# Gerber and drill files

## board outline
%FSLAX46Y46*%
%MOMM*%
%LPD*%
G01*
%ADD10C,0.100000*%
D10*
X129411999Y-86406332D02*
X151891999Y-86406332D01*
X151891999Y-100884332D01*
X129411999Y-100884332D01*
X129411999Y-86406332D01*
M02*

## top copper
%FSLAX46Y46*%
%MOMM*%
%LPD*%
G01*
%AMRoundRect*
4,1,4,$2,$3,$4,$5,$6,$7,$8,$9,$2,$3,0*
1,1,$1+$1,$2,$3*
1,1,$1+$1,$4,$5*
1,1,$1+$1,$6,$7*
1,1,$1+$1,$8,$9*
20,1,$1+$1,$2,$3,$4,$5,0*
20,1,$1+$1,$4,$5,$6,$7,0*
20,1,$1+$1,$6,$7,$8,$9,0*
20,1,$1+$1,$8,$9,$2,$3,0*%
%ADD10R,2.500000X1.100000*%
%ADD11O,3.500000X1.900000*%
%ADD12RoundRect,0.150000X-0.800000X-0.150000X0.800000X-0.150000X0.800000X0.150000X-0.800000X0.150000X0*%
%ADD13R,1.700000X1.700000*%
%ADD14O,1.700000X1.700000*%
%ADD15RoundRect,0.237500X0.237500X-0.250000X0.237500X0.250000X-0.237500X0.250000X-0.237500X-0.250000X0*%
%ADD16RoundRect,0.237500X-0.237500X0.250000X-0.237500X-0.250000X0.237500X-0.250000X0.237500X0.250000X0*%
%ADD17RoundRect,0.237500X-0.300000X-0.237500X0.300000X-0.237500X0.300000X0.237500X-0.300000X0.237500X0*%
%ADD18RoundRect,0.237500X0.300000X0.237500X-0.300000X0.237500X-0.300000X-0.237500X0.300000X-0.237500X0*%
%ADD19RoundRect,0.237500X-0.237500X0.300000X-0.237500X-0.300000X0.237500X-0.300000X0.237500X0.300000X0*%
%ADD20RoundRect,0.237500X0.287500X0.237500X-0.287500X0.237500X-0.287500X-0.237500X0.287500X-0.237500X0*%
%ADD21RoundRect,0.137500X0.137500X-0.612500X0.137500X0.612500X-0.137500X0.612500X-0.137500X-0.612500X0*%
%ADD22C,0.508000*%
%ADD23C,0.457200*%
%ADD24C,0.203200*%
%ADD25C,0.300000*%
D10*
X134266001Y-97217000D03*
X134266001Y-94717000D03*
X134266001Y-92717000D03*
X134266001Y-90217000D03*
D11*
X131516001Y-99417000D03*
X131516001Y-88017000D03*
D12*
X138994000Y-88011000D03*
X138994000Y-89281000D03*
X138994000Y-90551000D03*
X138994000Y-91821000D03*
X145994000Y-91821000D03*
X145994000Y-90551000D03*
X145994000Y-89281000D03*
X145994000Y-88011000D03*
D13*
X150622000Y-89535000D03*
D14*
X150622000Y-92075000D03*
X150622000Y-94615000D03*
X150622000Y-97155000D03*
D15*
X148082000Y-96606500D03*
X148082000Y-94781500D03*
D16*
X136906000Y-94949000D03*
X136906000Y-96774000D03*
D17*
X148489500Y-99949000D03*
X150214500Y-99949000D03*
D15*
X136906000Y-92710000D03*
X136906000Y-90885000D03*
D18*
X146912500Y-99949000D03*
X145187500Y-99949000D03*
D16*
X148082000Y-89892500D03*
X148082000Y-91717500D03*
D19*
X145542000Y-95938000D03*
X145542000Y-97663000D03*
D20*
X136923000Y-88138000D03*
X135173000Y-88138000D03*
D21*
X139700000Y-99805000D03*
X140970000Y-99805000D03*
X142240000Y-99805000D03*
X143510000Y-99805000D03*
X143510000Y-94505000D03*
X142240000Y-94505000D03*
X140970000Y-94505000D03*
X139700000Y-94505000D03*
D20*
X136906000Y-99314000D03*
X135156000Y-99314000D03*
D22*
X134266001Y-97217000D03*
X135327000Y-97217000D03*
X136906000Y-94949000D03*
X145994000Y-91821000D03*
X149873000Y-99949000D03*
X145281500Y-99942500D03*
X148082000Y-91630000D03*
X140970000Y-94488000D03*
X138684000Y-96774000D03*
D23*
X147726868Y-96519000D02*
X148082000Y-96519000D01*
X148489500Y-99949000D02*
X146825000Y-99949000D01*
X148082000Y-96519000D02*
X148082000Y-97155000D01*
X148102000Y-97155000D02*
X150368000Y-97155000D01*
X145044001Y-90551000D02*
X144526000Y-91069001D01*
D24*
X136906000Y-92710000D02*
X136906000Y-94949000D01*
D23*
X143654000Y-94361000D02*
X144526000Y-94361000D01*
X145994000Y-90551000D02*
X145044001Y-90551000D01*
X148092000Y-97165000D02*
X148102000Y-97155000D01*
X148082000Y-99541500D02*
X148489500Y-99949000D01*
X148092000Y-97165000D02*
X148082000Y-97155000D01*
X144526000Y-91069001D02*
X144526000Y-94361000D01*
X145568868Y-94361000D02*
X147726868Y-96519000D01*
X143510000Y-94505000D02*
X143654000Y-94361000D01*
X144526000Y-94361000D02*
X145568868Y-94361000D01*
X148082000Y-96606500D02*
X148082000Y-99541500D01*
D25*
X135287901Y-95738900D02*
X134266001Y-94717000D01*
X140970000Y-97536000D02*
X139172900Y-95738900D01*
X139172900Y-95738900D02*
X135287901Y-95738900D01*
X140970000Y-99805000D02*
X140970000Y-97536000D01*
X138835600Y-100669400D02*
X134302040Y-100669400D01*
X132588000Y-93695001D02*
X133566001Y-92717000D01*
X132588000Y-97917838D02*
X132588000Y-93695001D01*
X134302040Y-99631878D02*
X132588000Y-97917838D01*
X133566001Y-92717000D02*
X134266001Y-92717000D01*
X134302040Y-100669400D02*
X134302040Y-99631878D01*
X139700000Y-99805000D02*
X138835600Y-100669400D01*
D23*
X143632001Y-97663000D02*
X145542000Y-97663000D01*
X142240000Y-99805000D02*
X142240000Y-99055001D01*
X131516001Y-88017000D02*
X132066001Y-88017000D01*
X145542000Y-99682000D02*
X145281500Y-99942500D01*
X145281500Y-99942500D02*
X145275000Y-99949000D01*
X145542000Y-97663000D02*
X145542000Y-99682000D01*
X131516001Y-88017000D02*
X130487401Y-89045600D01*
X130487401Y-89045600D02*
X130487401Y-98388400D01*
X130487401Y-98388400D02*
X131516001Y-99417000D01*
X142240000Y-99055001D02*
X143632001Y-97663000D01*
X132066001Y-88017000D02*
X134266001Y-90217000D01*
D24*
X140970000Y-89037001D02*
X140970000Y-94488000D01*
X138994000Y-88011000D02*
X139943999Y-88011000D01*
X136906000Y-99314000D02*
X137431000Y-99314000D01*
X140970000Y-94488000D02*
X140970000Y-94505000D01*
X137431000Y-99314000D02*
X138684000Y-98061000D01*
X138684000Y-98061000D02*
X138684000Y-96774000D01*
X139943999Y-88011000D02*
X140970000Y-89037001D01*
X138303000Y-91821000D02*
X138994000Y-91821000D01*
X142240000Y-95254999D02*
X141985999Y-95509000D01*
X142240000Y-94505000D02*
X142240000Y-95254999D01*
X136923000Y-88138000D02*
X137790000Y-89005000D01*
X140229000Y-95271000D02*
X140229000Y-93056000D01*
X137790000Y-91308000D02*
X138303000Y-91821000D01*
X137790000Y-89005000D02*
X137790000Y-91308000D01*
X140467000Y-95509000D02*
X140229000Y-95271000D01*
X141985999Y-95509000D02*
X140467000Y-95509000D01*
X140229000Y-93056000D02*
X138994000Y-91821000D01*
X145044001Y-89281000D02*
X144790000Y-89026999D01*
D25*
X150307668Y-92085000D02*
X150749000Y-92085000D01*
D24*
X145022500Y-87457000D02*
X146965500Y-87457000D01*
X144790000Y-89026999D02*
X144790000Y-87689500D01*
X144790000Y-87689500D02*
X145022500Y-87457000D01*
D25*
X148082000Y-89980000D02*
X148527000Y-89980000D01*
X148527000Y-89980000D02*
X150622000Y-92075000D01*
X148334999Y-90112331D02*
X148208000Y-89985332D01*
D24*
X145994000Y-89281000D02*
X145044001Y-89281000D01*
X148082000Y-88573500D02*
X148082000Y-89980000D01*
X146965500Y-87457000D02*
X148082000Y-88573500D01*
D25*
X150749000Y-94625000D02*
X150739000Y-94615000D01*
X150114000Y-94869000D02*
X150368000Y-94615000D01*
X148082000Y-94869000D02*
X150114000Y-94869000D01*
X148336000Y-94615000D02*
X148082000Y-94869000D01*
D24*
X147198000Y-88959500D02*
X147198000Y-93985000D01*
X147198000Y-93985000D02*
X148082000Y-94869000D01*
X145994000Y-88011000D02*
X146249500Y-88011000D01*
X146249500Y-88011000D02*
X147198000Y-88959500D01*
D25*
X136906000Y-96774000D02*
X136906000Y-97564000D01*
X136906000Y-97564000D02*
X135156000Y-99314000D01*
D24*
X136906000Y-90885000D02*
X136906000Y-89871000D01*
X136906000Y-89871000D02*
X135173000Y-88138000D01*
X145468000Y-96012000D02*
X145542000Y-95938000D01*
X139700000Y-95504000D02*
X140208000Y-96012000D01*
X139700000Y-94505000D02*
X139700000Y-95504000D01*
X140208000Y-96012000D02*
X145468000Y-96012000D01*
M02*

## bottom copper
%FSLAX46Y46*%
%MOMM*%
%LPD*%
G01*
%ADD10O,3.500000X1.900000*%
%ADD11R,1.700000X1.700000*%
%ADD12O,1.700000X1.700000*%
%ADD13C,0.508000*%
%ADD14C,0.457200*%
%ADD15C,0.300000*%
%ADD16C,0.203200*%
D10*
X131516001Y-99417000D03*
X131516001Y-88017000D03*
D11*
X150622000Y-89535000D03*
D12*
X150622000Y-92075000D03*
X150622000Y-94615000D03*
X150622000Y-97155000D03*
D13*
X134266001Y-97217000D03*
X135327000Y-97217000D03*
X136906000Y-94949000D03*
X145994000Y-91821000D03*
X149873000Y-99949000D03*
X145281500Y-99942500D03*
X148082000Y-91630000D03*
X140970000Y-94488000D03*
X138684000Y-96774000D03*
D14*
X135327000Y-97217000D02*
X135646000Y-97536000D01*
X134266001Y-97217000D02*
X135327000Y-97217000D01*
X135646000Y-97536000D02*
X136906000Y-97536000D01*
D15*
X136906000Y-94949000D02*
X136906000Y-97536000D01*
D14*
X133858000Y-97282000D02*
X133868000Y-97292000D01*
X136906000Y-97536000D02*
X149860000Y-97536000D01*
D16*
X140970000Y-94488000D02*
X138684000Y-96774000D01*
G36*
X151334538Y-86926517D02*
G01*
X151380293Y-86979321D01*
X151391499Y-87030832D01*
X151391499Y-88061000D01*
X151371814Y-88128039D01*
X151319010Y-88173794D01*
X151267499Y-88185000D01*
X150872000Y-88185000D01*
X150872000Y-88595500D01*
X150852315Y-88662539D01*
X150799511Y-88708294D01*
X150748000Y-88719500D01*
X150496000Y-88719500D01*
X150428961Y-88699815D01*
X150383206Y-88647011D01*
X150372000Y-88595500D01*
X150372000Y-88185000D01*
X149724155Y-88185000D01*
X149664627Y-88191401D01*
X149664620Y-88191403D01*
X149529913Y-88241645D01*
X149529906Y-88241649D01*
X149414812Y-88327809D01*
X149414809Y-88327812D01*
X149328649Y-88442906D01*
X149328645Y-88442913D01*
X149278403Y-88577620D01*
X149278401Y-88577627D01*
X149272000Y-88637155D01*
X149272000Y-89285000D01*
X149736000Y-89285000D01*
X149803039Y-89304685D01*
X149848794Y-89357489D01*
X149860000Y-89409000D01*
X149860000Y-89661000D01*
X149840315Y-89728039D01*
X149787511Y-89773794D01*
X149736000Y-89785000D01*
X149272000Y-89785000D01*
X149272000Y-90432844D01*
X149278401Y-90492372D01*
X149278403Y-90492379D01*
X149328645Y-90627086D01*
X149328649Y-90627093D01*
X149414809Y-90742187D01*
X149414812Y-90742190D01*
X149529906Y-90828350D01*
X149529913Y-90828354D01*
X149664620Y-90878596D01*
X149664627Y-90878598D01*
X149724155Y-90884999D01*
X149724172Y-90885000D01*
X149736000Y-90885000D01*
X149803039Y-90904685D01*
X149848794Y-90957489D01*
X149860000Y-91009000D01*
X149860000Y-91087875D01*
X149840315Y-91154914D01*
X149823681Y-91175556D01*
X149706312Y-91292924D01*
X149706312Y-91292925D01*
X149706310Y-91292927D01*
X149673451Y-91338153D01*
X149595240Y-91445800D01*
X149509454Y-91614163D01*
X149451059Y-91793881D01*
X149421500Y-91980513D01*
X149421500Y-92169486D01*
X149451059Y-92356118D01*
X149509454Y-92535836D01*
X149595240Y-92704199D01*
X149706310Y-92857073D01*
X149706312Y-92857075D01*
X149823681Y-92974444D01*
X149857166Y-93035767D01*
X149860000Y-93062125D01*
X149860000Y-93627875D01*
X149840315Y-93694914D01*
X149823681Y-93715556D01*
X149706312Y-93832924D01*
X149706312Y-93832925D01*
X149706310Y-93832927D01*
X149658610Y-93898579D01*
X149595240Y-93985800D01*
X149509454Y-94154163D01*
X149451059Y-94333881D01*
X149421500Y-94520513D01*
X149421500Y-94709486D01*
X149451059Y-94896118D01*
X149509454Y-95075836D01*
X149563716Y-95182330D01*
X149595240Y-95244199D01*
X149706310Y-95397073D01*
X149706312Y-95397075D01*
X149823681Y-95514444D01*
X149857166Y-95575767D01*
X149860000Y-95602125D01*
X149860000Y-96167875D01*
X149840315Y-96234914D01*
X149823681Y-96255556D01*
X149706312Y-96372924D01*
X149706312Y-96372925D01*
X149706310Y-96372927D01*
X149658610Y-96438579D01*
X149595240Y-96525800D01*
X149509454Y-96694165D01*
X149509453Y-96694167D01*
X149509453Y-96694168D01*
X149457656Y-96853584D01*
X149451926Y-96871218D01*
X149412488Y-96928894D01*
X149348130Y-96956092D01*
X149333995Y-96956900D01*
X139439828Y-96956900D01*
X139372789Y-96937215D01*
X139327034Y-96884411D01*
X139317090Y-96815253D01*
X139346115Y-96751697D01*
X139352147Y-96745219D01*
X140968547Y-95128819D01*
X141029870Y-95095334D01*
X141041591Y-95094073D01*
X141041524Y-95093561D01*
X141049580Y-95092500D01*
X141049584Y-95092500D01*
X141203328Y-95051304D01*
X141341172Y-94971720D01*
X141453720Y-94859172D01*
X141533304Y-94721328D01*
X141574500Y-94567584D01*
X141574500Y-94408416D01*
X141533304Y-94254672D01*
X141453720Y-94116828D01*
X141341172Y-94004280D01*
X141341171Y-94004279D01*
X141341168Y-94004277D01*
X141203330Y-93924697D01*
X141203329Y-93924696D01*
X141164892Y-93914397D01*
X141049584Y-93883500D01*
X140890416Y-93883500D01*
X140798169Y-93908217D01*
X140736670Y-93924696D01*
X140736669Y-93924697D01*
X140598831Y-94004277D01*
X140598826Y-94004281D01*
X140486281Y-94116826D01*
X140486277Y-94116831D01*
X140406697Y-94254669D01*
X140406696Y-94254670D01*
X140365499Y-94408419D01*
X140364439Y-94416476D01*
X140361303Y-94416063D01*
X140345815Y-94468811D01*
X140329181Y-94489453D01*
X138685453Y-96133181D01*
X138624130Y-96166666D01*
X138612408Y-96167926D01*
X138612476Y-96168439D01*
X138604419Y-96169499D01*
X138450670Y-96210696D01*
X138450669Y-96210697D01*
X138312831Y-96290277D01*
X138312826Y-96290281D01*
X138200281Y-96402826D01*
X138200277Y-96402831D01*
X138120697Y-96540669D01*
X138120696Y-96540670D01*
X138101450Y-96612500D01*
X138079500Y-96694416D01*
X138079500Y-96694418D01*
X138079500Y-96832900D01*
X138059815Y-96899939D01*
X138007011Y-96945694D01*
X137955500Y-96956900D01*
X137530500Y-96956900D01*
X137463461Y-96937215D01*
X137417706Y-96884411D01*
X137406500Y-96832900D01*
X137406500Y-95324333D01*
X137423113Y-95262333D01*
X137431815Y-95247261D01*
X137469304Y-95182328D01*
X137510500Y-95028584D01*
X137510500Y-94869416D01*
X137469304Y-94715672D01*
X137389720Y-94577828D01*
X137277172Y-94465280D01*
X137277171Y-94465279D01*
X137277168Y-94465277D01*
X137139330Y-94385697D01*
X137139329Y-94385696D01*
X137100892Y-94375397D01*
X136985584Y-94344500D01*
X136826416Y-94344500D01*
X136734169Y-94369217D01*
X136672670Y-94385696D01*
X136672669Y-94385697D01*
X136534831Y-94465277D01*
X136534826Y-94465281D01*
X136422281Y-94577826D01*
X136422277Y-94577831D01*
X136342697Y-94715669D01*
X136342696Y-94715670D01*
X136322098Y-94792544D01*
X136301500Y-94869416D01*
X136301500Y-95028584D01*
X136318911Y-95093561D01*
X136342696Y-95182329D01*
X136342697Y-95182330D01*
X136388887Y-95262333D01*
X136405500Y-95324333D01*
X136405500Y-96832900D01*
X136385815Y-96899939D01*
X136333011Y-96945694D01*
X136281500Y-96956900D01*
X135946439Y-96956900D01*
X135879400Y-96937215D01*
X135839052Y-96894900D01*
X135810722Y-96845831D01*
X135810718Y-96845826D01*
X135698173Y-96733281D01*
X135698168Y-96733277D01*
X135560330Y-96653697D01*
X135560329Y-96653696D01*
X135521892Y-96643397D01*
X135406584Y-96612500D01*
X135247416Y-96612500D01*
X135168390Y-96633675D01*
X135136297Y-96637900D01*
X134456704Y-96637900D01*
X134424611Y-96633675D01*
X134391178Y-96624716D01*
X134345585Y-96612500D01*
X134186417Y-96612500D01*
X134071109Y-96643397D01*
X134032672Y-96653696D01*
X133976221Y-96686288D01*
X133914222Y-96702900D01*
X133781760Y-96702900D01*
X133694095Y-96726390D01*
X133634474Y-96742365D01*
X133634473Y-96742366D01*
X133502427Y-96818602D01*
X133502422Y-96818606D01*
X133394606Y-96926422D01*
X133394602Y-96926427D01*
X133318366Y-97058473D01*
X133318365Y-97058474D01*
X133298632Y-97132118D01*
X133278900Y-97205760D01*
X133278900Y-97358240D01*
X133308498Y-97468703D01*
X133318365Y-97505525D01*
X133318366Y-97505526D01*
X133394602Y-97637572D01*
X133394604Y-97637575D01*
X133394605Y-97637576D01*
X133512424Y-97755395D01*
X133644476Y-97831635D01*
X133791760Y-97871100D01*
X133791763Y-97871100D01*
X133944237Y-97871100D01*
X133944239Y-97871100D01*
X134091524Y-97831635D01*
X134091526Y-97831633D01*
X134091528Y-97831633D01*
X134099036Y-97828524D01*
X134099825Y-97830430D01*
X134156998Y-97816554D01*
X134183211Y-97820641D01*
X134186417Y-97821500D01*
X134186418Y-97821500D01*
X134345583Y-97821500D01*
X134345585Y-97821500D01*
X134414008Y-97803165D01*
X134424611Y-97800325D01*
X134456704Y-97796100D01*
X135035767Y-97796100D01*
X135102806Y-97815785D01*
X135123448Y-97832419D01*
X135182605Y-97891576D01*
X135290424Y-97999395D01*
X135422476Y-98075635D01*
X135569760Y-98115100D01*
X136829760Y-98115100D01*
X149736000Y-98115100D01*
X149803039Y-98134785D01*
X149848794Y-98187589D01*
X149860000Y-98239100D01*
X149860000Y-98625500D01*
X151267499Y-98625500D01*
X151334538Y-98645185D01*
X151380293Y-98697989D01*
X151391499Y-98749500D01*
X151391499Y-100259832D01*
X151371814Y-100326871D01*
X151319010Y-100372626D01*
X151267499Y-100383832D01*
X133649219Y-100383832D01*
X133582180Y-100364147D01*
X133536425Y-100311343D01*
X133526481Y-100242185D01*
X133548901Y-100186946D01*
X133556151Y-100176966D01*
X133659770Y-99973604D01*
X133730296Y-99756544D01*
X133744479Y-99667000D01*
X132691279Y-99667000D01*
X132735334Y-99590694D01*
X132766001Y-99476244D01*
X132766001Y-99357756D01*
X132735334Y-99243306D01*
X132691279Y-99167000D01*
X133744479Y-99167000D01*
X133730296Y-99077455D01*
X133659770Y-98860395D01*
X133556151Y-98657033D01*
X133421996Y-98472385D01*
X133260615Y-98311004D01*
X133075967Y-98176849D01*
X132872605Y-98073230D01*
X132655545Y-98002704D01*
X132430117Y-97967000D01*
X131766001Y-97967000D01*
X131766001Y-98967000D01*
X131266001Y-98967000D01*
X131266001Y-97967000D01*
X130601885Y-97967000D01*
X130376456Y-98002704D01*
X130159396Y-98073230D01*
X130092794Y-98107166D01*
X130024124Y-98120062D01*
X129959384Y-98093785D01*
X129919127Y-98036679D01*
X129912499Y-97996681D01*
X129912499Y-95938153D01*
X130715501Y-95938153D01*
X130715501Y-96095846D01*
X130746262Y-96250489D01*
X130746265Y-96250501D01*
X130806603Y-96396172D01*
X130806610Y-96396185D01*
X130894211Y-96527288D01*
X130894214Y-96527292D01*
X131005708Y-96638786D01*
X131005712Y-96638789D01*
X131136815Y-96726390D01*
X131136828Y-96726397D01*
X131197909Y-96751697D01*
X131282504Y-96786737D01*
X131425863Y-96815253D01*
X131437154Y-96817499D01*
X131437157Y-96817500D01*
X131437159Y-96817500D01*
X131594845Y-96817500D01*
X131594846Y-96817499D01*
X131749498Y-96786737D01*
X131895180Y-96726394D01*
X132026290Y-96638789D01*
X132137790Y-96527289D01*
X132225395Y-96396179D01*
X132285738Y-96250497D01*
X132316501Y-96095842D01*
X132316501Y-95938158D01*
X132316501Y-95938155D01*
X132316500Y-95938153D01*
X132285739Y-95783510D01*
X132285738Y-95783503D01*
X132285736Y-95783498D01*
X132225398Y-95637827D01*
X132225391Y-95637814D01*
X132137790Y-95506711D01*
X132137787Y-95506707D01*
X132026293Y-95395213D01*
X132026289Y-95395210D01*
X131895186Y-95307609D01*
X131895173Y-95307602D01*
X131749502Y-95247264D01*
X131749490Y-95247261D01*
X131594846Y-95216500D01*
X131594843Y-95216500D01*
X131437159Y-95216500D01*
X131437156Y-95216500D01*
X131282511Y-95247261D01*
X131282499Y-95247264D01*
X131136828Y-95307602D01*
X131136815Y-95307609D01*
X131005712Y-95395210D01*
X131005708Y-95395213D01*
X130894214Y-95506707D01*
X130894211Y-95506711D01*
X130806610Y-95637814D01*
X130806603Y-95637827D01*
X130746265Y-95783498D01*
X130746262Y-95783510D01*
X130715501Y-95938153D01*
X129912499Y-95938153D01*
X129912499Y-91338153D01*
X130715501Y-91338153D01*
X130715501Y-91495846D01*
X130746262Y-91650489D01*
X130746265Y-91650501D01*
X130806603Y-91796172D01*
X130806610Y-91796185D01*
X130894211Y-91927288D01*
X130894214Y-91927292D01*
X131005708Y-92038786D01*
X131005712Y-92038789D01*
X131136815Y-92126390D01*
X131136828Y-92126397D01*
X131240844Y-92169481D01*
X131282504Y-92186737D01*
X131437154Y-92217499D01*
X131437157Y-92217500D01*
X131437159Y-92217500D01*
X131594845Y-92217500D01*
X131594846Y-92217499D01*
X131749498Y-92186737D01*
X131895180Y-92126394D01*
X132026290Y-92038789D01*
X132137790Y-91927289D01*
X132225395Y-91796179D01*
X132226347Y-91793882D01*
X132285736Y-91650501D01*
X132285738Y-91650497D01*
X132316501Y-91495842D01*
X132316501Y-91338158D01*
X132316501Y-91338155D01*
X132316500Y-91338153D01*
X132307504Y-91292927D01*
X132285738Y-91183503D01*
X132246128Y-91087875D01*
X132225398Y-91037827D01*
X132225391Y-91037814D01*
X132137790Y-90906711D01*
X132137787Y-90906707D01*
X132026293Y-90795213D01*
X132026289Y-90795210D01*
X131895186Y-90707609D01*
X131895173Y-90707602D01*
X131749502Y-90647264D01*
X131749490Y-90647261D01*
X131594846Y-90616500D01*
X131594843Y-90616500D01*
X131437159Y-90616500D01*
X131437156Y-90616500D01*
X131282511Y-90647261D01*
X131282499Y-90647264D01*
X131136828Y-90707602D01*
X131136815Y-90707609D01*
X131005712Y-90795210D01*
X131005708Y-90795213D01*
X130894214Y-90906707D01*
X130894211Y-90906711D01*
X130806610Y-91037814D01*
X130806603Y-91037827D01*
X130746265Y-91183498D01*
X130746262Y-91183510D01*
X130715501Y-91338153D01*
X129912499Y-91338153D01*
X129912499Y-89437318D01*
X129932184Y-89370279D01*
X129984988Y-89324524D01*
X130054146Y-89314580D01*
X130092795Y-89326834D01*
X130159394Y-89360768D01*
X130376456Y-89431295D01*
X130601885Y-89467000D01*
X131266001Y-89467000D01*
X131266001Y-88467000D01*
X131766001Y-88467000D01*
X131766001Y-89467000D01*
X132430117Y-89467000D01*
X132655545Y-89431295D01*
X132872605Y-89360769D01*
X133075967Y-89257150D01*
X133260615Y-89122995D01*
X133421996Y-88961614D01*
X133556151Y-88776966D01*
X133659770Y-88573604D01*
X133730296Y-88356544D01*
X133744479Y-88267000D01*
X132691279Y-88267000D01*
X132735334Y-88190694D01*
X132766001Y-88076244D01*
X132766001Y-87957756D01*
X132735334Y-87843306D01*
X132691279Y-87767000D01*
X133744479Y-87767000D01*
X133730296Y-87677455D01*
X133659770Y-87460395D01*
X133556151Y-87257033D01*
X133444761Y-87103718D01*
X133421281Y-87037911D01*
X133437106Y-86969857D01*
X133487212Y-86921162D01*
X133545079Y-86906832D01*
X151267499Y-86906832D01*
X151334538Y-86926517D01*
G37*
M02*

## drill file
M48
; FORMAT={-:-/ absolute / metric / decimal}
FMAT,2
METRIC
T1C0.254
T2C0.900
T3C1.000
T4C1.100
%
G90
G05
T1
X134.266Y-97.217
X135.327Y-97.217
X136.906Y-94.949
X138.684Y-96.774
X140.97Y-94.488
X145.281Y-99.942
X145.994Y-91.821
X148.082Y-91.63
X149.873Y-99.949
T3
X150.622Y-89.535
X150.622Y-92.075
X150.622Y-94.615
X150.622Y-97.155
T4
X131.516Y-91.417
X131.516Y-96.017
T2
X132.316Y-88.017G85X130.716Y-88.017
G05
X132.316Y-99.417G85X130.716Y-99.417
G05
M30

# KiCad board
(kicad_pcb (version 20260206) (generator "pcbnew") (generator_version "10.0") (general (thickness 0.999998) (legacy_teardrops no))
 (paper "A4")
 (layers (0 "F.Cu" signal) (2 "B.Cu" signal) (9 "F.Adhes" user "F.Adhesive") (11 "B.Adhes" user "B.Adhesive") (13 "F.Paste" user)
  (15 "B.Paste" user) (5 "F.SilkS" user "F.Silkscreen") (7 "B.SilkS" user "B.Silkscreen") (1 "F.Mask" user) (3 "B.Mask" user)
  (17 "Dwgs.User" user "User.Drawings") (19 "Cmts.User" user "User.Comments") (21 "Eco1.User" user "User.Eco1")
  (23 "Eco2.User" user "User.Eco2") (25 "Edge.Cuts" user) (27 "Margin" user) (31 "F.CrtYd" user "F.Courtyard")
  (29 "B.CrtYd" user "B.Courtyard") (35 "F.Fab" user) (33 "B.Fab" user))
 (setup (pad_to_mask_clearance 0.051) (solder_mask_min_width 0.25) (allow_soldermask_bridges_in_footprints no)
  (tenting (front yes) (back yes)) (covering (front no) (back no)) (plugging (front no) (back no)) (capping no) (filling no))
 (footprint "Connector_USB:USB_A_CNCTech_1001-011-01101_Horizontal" (layer "F.Cu") (at 124.616001 93.717 180)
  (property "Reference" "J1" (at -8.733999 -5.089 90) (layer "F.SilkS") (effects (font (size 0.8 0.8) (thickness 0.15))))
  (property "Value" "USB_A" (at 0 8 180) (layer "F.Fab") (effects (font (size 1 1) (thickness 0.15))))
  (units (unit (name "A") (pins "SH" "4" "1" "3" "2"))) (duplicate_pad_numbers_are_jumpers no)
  (pad "" np_thru_hole circle (at -6.9 -2.3 180) (size 1.1 1.1) (drill 1.1) (layers "*.Cu" "*.Mask"))
  (pad "" np_thru_hole circle (at -6.9 2.3 180) (size 1.1 1.1) (drill 1.1) (layers "*.Cu" "*.Mask"))
  (pad "1" smd rect (at -9.65 -3.5 180) (size 2.5 1.1) (layers "F.Cu" "F.Mask" "F.Paste") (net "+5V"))
  (pad "2" smd rect (at -9.65 -1 180) (size 2.5 1.1) (layers "F.Cu" "F.Mask" "F.Paste") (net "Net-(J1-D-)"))
  (pad "3" smd rect (at -9.65 1 180) (size 2.5 1.1) (layers "F.Cu" "F.Mask" "F.Paste") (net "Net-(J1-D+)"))
  (pad "4" smd rect (at -9.65 3.5 180) (size 2.5 1.1) (layers "F.Cu" "F.Mask" "F.Paste") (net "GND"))
  (pad "SH" thru_hole oval (at -6.9 -5.7 180) (size 3.5 1.9) (drill oval 2.5 0.9) (layers "*.Cu" "*.Mask") (remove_unused_layers no)
   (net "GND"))
  (pad "SH" thru_hole oval (at -6.9 5.7 180) (size 3.5 1.9) (drill oval 2.5 0.9) (layers "*.Cu" "*.Mask") (remove_unused_layers no)
   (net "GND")))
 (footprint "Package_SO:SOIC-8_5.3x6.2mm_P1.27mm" (layer "F.Cu") (at 142.494 89.916)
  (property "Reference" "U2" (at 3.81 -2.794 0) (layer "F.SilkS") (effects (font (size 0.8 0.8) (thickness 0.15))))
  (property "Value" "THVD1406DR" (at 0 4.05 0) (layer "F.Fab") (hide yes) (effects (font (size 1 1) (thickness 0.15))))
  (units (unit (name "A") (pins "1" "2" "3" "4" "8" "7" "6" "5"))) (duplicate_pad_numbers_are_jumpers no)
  (pad "1" smd roundrect (at -3.5 -1.905) (size 1.9 0.6) (layers "F.Cu" "F.Mask" "F.Paste") (roundrect_rratio 0.25) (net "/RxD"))
  (pad "2" smd roundrect (at -3.5 -0.635) (size 1.9 0.6) (layers "F.Cu" "F.Mask" "F.Paste") (roundrect_rratio 0.25)
   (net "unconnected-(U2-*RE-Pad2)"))
  (pad "3" smd roundrect (at -3.5 0.635) (size 1.9 0.6) (layers "F.Cu" "F.Mask" "F.Paste") (roundrect_rratio 0.25)
   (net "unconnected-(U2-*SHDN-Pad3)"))
  (pad "4" smd roundrect (at -3.5 1.905) (size 1.9 0.6) (layers "F.Cu" "F.Mask" "F.Paste") (roundrect_rratio 0.25) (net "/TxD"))
  (pad "5" smd roundrect (at 3.5 1.905) (size 1.9 0.6) (layers "F.Cu" "F.Mask" "F.Paste") (roundrect_rratio 0.25) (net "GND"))
  (pad "6" smd roundrect (at 3.5 0.635) (size 1.9 0.6) (layers "F.Cu" "F.Mask" "F.Paste") (roundrect_rratio 0.25) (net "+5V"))
  (pad "7" smd roundrect (at 3.5 -0.635) (size 1.9 0.6) (layers "F.Cu" "F.Mask" "F.Paste") (roundrect_rratio 0.25) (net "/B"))
  (pad "8" smd roundrect (at 3.5 -1.905) (size 1.9 0.6) (layers "F.Cu" "F.Mask" "F.Paste") (roundrect_rratio 0.25) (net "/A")))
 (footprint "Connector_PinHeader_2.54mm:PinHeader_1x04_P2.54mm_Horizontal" (layer "F.Cu") (at 150.622 89.535)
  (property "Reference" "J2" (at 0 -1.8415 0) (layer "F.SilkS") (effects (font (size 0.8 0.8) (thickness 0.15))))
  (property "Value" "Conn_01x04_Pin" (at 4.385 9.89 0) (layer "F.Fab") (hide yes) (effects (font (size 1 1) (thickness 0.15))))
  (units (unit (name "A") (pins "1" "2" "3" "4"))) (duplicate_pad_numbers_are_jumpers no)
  (pad "1" thru_hole rect (at 0 0) (size 1.7 1.7) (drill 1) (layers "*.Cu" "*.Mask") (remove_unused_layers no) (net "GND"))
  (pad "2" thru_hole oval (at 0 2.54) (size 1.7 1.7) (drill 1) (layers "*.Cu" "*.Mask") (remove_unused_layers no) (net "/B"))
  (pad "3" thru_hole oval (at 0 5.08) (size 1.7 1.7) (drill 1) (layers "*.Cu" "*.Mask") (remove_unused_layers no) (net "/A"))
  (pad "4" thru_hole oval (at 0 7.62) (size 1.7 1.7) (drill 1) (layers "*.Cu" "*.Mask") (remove_unused_layers no) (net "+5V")))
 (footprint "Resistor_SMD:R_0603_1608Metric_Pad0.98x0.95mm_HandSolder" (layer "F.Cu") (at 148.082 95.694 90)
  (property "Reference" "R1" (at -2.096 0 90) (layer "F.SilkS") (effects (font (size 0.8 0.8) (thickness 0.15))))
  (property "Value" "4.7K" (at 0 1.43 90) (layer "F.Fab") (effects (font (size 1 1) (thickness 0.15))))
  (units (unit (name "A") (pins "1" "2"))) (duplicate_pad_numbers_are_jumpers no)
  (pad "1" smd roundrect (at -0.9125 0 90) (size 0.975 0.95) (layers "F.Cu" "F.Mask" "F.Paste") (roundrect_rratio 0.25) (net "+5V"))
  (pad "2" smd roundrect (at 0.9125 0 90) (size 0.975 0.95) (layers "F.Cu" "F.Mask" "F.Paste") (roundrect_rratio 0.25) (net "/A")))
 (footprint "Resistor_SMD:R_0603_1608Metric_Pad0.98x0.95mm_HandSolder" (layer "F.Cu") (at 136.906 95.8615 -90)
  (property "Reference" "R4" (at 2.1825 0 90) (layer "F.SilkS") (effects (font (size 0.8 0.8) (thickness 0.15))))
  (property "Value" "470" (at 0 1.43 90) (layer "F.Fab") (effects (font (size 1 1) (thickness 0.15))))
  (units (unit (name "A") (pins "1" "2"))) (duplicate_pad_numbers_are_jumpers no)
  (pad "1" smd roundrect (at -0.9125 0 270) (size 0.975 0.95) (layers "F.Cu" "F.Mask" "F.Paste") (roundrect_rratio 0.25) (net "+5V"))
  (pad "2" smd roundrect (at 0.9125 0 270) (size 0.975 0.95) (layers "F.Cu" "F.Mask" "F.Paste") (roundrect_rratio 0.25) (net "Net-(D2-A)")))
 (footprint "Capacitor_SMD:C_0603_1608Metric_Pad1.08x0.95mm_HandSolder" (layer "F.Cu") (at 149.352 99.949)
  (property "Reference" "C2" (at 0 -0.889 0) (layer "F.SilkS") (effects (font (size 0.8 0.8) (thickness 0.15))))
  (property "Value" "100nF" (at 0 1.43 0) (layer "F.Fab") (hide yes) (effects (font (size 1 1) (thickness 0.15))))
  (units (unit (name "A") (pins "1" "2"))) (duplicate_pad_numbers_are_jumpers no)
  (pad "1" smd roundrect (at -0.8625 0) (size 1.075 0.95) (layers "F.Cu" "F.Mask" "F.Paste") (roundrect_rratio 0.25) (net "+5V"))
  (pad "2" smd roundrect (at 0.8625 0) (size 1.075 0.95) (layers "F.Cu" "F.Mask" "F.Paste") (roundrect_rratio 0.25) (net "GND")))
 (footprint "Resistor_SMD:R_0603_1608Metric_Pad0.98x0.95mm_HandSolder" (layer "F.Cu") (at 136.906 91.7975 90)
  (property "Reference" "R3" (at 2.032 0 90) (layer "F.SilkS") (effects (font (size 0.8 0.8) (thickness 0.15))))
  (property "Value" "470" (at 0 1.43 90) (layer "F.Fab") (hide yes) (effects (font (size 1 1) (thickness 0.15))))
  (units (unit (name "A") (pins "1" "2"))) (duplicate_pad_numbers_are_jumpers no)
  (pad "1" smd roundrect (at -0.9125 0 90) (size 0.975 0.95) (layers "F.Cu" "F.Mask" "F.Paste") (roundrect_rratio 0.25) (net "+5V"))
  (pad "2" smd roundrect (at 0.9125 0 90) (size 0.975 0.95) (layers "F.Cu" "F.Mask" "F.Paste") (roundrect_rratio 0.25) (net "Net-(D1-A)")))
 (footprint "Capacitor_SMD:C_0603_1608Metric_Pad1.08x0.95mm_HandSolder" (layer "F.Cu") (at 146.05 99.949 180)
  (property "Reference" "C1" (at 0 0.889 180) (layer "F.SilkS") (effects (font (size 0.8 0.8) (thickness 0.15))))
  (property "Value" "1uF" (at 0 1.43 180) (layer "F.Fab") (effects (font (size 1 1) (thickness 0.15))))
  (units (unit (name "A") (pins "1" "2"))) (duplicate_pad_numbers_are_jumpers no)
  (pad "1" smd roundrect (at -0.8625 0 180) (size 1.075 0.95) (layers "F.Cu" "F.Mask" "F.Paste") (roundrect_rratio 0.25) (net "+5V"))
  (pad "2" smd roundrect (at 0.8625 0 180) (size 1.075 0.95) (layers "F.Cu" "F.Mask" "F.Paste") (roundrect_rratio 0.25) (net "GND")))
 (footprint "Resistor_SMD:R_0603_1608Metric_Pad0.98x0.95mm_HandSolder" (layer "F.Cu") (at 148.082 90.805 -90)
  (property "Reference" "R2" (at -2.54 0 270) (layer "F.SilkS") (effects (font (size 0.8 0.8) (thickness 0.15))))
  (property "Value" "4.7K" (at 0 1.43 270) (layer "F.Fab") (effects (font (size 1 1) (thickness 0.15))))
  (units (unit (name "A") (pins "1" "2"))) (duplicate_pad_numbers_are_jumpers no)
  (pad "1" smd roundrect (at -0.9125 0 270) (size 0.975 0.95) (layers "F.Cu" "F.Mask" "F.Paste") (roundrect_rratio 0.25) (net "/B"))
  (pad "2" smd roundrect (at 0.9125 0 270) (size 0.975 0.95) (layers "F.Cu" "F.Mask" "F.Paste") (roundrect_rratio 0.25) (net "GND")))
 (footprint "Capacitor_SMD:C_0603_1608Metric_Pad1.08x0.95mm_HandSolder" (layer "F.Cu") (at 145.542 96.8005 -90)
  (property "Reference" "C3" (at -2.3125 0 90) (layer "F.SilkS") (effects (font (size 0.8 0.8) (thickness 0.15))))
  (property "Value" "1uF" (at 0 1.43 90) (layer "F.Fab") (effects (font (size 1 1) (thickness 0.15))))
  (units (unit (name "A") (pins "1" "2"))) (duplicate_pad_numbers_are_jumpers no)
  (pad "1" smd roundrect (at -0.8625 0 270) (size 1.075 0.95) (layers "F.Cu" "F.Mask" "F.Paste") (roundrect_rratio 0.25) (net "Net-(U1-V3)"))
  (pad "2" smd roundrect (at 0.8625 0 270) (size 1.075 0.95) (layers "F.Cu" "F.Mask" "F.Paste") (roundrect_rratio 0.25) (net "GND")))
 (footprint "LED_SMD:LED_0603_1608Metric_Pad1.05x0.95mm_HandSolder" (layer "F.Cu") (at 136.048 88.138 180)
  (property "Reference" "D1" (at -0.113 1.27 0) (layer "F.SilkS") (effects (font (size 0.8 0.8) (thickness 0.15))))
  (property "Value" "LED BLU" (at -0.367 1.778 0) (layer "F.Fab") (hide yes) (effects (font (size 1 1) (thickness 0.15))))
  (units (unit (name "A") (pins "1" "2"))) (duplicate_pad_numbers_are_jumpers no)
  (pad "1" smd roundrect (at -0.875 0 180) (size 1.05 0.95) (layers "F.Cu" "F.Mask" "F.Paste") (roundrect_rratio 0.25) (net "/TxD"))
  (pad "2" smd roundrect (at 0.875 0 180) (size 1.05 0.95) (layers "F.Cu" "F.Mask" "F.Paste") (roundrect_rratio 0.25) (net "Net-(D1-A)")))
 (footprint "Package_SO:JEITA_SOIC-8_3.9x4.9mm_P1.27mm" (layer "F.Cu") (at 141.605 97.155 90)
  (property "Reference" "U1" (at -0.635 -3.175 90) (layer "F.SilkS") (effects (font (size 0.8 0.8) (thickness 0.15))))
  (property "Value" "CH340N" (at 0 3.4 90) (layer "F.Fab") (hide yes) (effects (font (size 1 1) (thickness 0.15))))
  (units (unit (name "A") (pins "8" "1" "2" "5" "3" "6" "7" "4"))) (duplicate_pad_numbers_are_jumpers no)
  (pad "1" smd roundrect (at -2.65 -1.905 90) (size 1.5 0.55) (layers "F.Cu" "F.Mask" "F.Paste") (roundrect_rratio 0.25) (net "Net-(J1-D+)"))
  (pad "2" smd roundrect (at -2.65 -0.635 90) (size 1.5 0.55) (layers "F.Cu" "F.Mask" "F.Paste") (roundrect_rratio 0.25) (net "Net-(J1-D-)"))
  (pad "3" smd roundrect (at -2.65 0.635 90) (size 1.5 0.55) (layers "F.Cu" "F.Mask" "F.Paste") (roundrect_rratio 0.25) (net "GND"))
  (pad "4" smd roundrect (at -2.65 1.905 90) (size 1.5 0.55) (layers "F.Cu" "F.Mask" "F.Paste") (roundrect_rratio 0.25)
   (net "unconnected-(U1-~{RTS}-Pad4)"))
  (pad "5" smd roundrect (at 2.65 1.905 90) (size 1.5 0.55) (layers "F.Cu" "F.Mask" "F.Paste") (roundrect_rratio 0.25) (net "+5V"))
  (pad "6" smd roundrect (at 2.65 0.635 90) (size 1.5 0.55) (layers "F.Cu" "F.Mask" "F.Paste") (roundrect_rratio 0.25) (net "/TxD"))
  (pad "7" smd roundrect (at 2.65 -0.635 90) (size 1.5 0.55) (layers "F.Cu" "F.Mask" "F.Paste") (roundrect_rratio 0.25) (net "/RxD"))
  (pad "8" smd roundrect (at 2.65 -1.905 90) (size 1.5 0.55) (layers "F.Cu" "F.Mask" "F.Paste") (roundrect_rratio 0.25) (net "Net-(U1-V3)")))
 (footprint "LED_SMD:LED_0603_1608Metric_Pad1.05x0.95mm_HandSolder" (layer "F.Cu") (at 136.031 99.314 180)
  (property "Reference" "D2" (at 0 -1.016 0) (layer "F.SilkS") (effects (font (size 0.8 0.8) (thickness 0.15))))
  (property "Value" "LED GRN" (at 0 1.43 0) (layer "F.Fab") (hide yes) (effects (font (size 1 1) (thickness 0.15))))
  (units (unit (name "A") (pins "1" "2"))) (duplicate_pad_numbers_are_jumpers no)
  (pad "1" smd roundrect (at -0.875 0 180) (size 1.05 0.95) (layers "F.Cu" "F.Mask" "F.Paste") (roundrect_rratio 0.25) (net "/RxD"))
  (pad "2" smd roundrect (at 0.875 0 180) (size 1.05 0.95) (layers "F.Cu" "F.Mask" "F.Paste") (roundrect_rratio 0.25) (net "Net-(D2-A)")))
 (gr_rect (start 129.411999 86.406332) (end 151.891999 100.884332) (stroke (width 0.1) (type solid)) (fill no) (layer "Edge.Cuts"))
 (segment (start 147.726868 96.519) (end 148.082 96.519) (width 0.4572) (layer "F.Cu") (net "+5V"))
 (segment (start 148.4895 99.949) (end 146.825 99.949) (width 0.4572) (layer "F.Cu") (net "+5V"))
 (segment (start 148.082 96.519) (end 148.082 97.155) (width 0.4572) (layer "F.Cu") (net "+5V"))
 (segment (start 148.102 97.155) (end 150.368 97.155) (width 0.4572) (layer "F.Cu") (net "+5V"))
 (segment (start 145.044001 90.551) (end 144.526 91.069001) (width 0.4572) (layer "F.Cu") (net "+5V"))
 (segment (start 136.906 92.71) (end 136.906 94.949) (width 0.2032) (layer "F.Cu") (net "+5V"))
 (segment (start 143.654 94.361) (end 144.526 94.361) (width 0.4572) (layer "F.Cu") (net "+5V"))
 (segment (start 145.994 90.551) (end 145.044001 90.551) (width 0.4572) (layer "F.Cu") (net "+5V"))
 (segment (start 148.092 97.165) (end 148.102 97.155) (width 0.4572) (layer "F.Cu") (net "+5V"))
 (segment (start 148.082 99.5415) (end 148.4895 99.949) (width 0.4572) (layer "F.Cu") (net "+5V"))
 (segment (start 148.092 97.165) (end 148.082 97.155) (width 0.4572) (layer "F.Cu") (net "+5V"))
 (segment (start 144.526 91.069001) (end 144.526 94.361) (width 0.4572) (layer "F.Cu") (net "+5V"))
 (segment (start 145.568868 94.361) (end 147.726868 96.519) (width 0.4572) (layer "F.Cu") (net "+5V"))
 (segment (start 143.51 94.505) (end 143.654 94.361) (width 0.4572) (layer "F.Cu") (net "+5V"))
 (segment (start 144.526 94.361) (end 145.568868 94.361) (width 0.4572) (layer "F.Cu") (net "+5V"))
 (segment (start 148.082 96.6065) (end 148.082 99.5415) (width 0.4572) (layer "F.Cu") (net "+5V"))
 (via (at 134.266001 97.217) (size 0.508) (drill 0.254) (layers "F.Cu" "B.Cu") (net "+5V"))
 (via (at 135.327 97.217) (size 0.508) (drill 0.254) (layers "F.Cu" "B.Cu") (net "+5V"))
 (via (at 136.906 94.949) (size 0.508) (drill 0.254) (layers "F.Cu" "B.Cu") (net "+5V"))
 (segment (start 135.327 97.217) (end 135.646 97.536) (width 0.4572) (layer "B.Cu") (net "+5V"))
 (segment (start 134.266001 97.217) (end 135.327 97.217) (width 0.4572) (layer "B.Cu") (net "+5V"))
 (segment (start 135.646 97.536) (end 136.906 97.536) (width 0.4572) (layer "B.Cu") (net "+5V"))
 (segment (start 136.906 94.949) (end 136.906 97.536) (width 0.3) (layer "B.Cu") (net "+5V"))
 (segment (start 133.858 97.282) (end 133.868 97.292) (width 0.4572) (layer "B.Cu") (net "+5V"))
 (segment (start 136.906 97.536) (end 149.86 97.536) (width 0.4572) (layer "B.Cu") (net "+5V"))
 (segment (start 135.287901 95.7389) (end 134.266001 94.717) (width 0.3) (layer "F.Cu") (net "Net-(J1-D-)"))
 (segment (start 140.97 97.536) (end 139.1729 95.7389) (width 0.3) (layer "F.Cu") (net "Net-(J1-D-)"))
 (segment (start 139.1729 95.7389) (end 135.287901 95.7389) (width 0.3) (layer "F.Cu") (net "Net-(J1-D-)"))
 (segment (start 140.97 99.805) (end 140.97 97.536) (width 0.3) (layer "F.Cu") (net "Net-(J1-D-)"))
 (segment (start 138.8356 100.6694) (end 134.30204 100.6694) (width 0.3) (layer "F.Cu") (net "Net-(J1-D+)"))
 (segment (start 132.588 93.695001) (end 133.566001 92.717) (width 0.3) (layer "F.Cu") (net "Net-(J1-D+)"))
 (segment (start 132.588 97.917838) (end 132.588 93.695001) (width 0.3) (layer "F.Cu") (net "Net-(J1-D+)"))
 (segment (start 134.30204 99.631878) (end 132.588 97.917838) (width 0.3) (layer "F.Cu") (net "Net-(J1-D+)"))
 (segment (start 133.566001 92.717) (end 134.266001 92.717) (width 0.3) (layer "F.Cu") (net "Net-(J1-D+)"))
 (segment (start 134.30204 100.6694) (end 134.30204 99.631878) (width 0.3) (layer "F.Cu") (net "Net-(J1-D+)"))
 (segment (start 139.7 99.805) (end 138.8356 100.6694) (width 0.3) (layer "F.Cu") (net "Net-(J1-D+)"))
 (segment (start 143.632001 97.663) (end 145.542 97.663) (width 0.4572) (layer "F.Cu") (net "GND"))
 (segment (start 142.24 99.805) (end 142.24 99.055001) (width 0.4572) (layer "F.Cu") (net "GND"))
 (segment (start 131.516001 88.017) (end 132.066001 88.017) (width 0.4572) (layer "F.Cu") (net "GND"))
 (segment (start 145.542 99.682) (end 145.2815 99.9425) (width 0.4572) (layer "F.Cu") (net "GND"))
 (segment (start 145.2815 99.9425) (end 145.275 99.949) (width 0.4572) (layer "F.Cu") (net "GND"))
 (segment (start 145.542 97.663) (end 145.542 99.682) (width 0.4572) (layer "F.Cu") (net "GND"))
 (segment (start 131.516001 88.017) (end 130.487401 89.0456) (width 0.4572) (layer "F.Cu") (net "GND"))
 (segment (start 130.487401 89.0456) (end 130.487401 98.3884) (width 0.4572) (layer "F.Cu") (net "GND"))
 (segment (start 130.487401 98.3884) (end 131.516001 99.417) (width 0.4572) (layer "F.Cu") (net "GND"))
 (segment (start 142.24 99.055001) (end 143.632001 97.663) (width 0.4572) (layer "F.Cu") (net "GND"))
 (segment (start 132.066001 88.017) (end 134.266001 90.217) (width 0.4572) (layer "F.Cu") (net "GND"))
 (via (at 145.994 91.821) (size 0.508) (drill 0.254) (layers "F.Cu" "B.Cu") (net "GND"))
 (via (at 149.873 99.949) (size 0.508) (drill 0.254) (layers "F.Cu" "B.Cu") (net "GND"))
 (via (at 145.2815 99.9425) (size 0.508) (drill 0.254) (layers "F.Cu" "B.Cu") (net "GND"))
 (via (at 148.082 91.63) (size 0.508) (drill 0.254) (layers "F.Cu" "B.Cu") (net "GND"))
 (segment (start 140.97 89.037001) (end 140.97 94.488) (width 0.2032) (layer "F.Cu") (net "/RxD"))
 (segment (start 138.994 88.011) (end 139.943999 88.011) (width 0.2032) (layer "F.Cu") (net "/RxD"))
 (segment (start 136.906 99.314) (end 137.431 99.314) (width 0.2032) (layer "F.Cu") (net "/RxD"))
 (segment (start 140.97 94.488) (end 140.97 94.505) (width 0.2032) (layer "F.Cu") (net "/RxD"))
 (segment (start 137.431 99.314) (end 138.684 98.061) (width 0.2032) (layer "F.Cu") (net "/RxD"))
 (segment (start 138.684 98.061) (end 138.684 96.774) (width 0.2032) (layer "F.Cu") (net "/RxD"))
 (segment (start 139.943999 88.011) (end 140.97 89.037001) (width 0.2032) (layer "F.Cu") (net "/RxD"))
 (via (at 140.97 94.488) (size 0.508) (drill 0.254) (layers "F.Cu" "B.Cu") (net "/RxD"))
 (via (at 138.684 96.774) (size 0.508) (drill 0.254) (layers "F.Cu" "B.Cu") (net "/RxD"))
 (segment (start 140.97 94.488) (end 138.684 96.774) (width 0.2032) (layer "B.Cu") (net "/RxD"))
 (segment (start 138.303 91.821) (end 138.994 91.821) (width 0.2032) (layer "F.Cu") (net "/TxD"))
 (segment (start 142.24 95.254999) (end 141.985999 95.509) (width 0.2032) (layer "F.Cu") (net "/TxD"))
 (segment (start 142.24 94.505) (end 142.24 95.254999) (width 0.2032) (layer "F.Cu") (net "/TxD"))
 (segment (start 136.923 88.138) (end 137.79 89.005) (width 0.2032) (layer "F.Cu") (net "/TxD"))
 (segment (start 140.229 95.271) (end 140.229 93.056) (width 0.2032) (layer "F.Cu") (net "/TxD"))
 (segment (start 137.79 91.308) (end 138.303 91.821) (width 0.2032) (layer "F.Cu") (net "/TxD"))
 (segment (start 137.79 89.005) (end 137.79 91.308) (width 0.2032) (layer "F.Cu") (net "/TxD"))
 (segment (start 140.467 95.509) (end 140.229 95.271) (width 0.2032) (layer "F.Cu") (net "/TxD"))
 (segment (start 141.985999 95.509) (end 140.467 95.509) (width 0.2032) (layer "F.Cu") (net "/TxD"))
 (segment (start 140.229 93.056) (end 138.994 91.821) (width 0.2032) (layer "F.Cu") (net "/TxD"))
 (segment (start 145.044001 89.281) (end 144.79 89.026999) (width 0.2032) (layer "F.Cu") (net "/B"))
 (segment (start 150.307668 92.085) (end 150.749 92.085) (width 0.3) (layer "F.Cu") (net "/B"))
 (segment (start 145.0225 87.457) (end 146.9655 87.457) (width 0.2032) (layer "F.Cu") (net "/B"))
 (segment (start 144.79 89.026999) (end 144.79 87.6895) (width 0.2032) (layer "F.Cu") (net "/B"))
 (segment (start 144.79 87.6895) (end 145.0225 87.457) (width 0.2032) (layer "F.Cu") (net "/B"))
 (segment (start 148.082 89.98) (end 148.527 89.98) (width 0.3) (layer "F.Cu") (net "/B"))
 (segment (start 148.527 89.98) (end 150.622 92.075) (width 0.3) (layer "F.Cu") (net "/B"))
 (segment (start 148.334999 90.112331) (end 148.208 89.985332) (width 0.3) (layer "F.Cu") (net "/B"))
 (segment (start 145.994 89.281) (end 145.044001 89.281) (width 0.2032) (layer "F.Cu") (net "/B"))
 (segment (start 148.082 88.5735) (end 148.082 89.98) (width 0.2032) (layer "F.Cu") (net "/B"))
 (segment (start 146.9655 87.457) (end 148.082 88.5735) (width 0.2032) (layer "F.Cu") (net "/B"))
 (segment (start 150.749 94.625) (end 150.739 94.615) (width 0.3) (layer "F.Cu") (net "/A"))
 (segment (start 150.114 94.869) (end 150.368 94.615) (width 0.3) (layer "F.Cu") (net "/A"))
 (segment (start 148.082 94.869) (end 150.114 94.869) (width 0.3) (layer "F.Cu") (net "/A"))
 (segment (start 148.336 94.615) (end 148.082 94.869) (width 0.3) (layer "F.Cu") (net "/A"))
 (segment (start 147.198 88.9595) (end 147.198 93.985) (width 0.2032) (layer "F.Cu") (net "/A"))
 (segment (start 147.198 93.985) (end 148.082 94.869) (width 0.2032) (layer "F.Cu") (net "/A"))
 (segment (start 145.994 88.011) (end 146.2495 88.011) (width 0.2032) (layer "F.Cu") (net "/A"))
 (segment (start 146.2495 88.011) (end 147.198 88.9595) (width 0.2032) (layer "F.Cu") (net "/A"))
 (segment (start 136.906 96.774) (end 136.906 97.564) (width 0.3) (layer "F.Cu") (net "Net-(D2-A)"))
 (segment (start 136.906 97.564) (end 135.156 99.314) (width 0.3) (layer "F.Cu") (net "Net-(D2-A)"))
 (segment (start 136.906 90.885) (end 136.906 89.871) (width 0.2032) (layer "F.Cu") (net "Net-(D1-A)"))
 (segment (start 136.906 89.871) (end 135.173 88.138) (width 0.2032) (layer "F.Cu") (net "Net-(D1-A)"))
 (segment (start 145.468 96.012) (end 145.542 95.938) (width 0.2032) (layer "F.Cu") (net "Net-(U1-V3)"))
 (segment (start 139.7 95.504) (end 140.208 96.012) (width 0.2032) (layer "F.Cu") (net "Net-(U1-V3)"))
 (segment (start 139.7 94.505) (end 139.7 95.504) (width 0.2032) (layer "F.Cu") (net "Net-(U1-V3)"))
 (segment (start 140.208 96.012) (end 145.468 96.012) (width 0.2032) (layer "F.Cu") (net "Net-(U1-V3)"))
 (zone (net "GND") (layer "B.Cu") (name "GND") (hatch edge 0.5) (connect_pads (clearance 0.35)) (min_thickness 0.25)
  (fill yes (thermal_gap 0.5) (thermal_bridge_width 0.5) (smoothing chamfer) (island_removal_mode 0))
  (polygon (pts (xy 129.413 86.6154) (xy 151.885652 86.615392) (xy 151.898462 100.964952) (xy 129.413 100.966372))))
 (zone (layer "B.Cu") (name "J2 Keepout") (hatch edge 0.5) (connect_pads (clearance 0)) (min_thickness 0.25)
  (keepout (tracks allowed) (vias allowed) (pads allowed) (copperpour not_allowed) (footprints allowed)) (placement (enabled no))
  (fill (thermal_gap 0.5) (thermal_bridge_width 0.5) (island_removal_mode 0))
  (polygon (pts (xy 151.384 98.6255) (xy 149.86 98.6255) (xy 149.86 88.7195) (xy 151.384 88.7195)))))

